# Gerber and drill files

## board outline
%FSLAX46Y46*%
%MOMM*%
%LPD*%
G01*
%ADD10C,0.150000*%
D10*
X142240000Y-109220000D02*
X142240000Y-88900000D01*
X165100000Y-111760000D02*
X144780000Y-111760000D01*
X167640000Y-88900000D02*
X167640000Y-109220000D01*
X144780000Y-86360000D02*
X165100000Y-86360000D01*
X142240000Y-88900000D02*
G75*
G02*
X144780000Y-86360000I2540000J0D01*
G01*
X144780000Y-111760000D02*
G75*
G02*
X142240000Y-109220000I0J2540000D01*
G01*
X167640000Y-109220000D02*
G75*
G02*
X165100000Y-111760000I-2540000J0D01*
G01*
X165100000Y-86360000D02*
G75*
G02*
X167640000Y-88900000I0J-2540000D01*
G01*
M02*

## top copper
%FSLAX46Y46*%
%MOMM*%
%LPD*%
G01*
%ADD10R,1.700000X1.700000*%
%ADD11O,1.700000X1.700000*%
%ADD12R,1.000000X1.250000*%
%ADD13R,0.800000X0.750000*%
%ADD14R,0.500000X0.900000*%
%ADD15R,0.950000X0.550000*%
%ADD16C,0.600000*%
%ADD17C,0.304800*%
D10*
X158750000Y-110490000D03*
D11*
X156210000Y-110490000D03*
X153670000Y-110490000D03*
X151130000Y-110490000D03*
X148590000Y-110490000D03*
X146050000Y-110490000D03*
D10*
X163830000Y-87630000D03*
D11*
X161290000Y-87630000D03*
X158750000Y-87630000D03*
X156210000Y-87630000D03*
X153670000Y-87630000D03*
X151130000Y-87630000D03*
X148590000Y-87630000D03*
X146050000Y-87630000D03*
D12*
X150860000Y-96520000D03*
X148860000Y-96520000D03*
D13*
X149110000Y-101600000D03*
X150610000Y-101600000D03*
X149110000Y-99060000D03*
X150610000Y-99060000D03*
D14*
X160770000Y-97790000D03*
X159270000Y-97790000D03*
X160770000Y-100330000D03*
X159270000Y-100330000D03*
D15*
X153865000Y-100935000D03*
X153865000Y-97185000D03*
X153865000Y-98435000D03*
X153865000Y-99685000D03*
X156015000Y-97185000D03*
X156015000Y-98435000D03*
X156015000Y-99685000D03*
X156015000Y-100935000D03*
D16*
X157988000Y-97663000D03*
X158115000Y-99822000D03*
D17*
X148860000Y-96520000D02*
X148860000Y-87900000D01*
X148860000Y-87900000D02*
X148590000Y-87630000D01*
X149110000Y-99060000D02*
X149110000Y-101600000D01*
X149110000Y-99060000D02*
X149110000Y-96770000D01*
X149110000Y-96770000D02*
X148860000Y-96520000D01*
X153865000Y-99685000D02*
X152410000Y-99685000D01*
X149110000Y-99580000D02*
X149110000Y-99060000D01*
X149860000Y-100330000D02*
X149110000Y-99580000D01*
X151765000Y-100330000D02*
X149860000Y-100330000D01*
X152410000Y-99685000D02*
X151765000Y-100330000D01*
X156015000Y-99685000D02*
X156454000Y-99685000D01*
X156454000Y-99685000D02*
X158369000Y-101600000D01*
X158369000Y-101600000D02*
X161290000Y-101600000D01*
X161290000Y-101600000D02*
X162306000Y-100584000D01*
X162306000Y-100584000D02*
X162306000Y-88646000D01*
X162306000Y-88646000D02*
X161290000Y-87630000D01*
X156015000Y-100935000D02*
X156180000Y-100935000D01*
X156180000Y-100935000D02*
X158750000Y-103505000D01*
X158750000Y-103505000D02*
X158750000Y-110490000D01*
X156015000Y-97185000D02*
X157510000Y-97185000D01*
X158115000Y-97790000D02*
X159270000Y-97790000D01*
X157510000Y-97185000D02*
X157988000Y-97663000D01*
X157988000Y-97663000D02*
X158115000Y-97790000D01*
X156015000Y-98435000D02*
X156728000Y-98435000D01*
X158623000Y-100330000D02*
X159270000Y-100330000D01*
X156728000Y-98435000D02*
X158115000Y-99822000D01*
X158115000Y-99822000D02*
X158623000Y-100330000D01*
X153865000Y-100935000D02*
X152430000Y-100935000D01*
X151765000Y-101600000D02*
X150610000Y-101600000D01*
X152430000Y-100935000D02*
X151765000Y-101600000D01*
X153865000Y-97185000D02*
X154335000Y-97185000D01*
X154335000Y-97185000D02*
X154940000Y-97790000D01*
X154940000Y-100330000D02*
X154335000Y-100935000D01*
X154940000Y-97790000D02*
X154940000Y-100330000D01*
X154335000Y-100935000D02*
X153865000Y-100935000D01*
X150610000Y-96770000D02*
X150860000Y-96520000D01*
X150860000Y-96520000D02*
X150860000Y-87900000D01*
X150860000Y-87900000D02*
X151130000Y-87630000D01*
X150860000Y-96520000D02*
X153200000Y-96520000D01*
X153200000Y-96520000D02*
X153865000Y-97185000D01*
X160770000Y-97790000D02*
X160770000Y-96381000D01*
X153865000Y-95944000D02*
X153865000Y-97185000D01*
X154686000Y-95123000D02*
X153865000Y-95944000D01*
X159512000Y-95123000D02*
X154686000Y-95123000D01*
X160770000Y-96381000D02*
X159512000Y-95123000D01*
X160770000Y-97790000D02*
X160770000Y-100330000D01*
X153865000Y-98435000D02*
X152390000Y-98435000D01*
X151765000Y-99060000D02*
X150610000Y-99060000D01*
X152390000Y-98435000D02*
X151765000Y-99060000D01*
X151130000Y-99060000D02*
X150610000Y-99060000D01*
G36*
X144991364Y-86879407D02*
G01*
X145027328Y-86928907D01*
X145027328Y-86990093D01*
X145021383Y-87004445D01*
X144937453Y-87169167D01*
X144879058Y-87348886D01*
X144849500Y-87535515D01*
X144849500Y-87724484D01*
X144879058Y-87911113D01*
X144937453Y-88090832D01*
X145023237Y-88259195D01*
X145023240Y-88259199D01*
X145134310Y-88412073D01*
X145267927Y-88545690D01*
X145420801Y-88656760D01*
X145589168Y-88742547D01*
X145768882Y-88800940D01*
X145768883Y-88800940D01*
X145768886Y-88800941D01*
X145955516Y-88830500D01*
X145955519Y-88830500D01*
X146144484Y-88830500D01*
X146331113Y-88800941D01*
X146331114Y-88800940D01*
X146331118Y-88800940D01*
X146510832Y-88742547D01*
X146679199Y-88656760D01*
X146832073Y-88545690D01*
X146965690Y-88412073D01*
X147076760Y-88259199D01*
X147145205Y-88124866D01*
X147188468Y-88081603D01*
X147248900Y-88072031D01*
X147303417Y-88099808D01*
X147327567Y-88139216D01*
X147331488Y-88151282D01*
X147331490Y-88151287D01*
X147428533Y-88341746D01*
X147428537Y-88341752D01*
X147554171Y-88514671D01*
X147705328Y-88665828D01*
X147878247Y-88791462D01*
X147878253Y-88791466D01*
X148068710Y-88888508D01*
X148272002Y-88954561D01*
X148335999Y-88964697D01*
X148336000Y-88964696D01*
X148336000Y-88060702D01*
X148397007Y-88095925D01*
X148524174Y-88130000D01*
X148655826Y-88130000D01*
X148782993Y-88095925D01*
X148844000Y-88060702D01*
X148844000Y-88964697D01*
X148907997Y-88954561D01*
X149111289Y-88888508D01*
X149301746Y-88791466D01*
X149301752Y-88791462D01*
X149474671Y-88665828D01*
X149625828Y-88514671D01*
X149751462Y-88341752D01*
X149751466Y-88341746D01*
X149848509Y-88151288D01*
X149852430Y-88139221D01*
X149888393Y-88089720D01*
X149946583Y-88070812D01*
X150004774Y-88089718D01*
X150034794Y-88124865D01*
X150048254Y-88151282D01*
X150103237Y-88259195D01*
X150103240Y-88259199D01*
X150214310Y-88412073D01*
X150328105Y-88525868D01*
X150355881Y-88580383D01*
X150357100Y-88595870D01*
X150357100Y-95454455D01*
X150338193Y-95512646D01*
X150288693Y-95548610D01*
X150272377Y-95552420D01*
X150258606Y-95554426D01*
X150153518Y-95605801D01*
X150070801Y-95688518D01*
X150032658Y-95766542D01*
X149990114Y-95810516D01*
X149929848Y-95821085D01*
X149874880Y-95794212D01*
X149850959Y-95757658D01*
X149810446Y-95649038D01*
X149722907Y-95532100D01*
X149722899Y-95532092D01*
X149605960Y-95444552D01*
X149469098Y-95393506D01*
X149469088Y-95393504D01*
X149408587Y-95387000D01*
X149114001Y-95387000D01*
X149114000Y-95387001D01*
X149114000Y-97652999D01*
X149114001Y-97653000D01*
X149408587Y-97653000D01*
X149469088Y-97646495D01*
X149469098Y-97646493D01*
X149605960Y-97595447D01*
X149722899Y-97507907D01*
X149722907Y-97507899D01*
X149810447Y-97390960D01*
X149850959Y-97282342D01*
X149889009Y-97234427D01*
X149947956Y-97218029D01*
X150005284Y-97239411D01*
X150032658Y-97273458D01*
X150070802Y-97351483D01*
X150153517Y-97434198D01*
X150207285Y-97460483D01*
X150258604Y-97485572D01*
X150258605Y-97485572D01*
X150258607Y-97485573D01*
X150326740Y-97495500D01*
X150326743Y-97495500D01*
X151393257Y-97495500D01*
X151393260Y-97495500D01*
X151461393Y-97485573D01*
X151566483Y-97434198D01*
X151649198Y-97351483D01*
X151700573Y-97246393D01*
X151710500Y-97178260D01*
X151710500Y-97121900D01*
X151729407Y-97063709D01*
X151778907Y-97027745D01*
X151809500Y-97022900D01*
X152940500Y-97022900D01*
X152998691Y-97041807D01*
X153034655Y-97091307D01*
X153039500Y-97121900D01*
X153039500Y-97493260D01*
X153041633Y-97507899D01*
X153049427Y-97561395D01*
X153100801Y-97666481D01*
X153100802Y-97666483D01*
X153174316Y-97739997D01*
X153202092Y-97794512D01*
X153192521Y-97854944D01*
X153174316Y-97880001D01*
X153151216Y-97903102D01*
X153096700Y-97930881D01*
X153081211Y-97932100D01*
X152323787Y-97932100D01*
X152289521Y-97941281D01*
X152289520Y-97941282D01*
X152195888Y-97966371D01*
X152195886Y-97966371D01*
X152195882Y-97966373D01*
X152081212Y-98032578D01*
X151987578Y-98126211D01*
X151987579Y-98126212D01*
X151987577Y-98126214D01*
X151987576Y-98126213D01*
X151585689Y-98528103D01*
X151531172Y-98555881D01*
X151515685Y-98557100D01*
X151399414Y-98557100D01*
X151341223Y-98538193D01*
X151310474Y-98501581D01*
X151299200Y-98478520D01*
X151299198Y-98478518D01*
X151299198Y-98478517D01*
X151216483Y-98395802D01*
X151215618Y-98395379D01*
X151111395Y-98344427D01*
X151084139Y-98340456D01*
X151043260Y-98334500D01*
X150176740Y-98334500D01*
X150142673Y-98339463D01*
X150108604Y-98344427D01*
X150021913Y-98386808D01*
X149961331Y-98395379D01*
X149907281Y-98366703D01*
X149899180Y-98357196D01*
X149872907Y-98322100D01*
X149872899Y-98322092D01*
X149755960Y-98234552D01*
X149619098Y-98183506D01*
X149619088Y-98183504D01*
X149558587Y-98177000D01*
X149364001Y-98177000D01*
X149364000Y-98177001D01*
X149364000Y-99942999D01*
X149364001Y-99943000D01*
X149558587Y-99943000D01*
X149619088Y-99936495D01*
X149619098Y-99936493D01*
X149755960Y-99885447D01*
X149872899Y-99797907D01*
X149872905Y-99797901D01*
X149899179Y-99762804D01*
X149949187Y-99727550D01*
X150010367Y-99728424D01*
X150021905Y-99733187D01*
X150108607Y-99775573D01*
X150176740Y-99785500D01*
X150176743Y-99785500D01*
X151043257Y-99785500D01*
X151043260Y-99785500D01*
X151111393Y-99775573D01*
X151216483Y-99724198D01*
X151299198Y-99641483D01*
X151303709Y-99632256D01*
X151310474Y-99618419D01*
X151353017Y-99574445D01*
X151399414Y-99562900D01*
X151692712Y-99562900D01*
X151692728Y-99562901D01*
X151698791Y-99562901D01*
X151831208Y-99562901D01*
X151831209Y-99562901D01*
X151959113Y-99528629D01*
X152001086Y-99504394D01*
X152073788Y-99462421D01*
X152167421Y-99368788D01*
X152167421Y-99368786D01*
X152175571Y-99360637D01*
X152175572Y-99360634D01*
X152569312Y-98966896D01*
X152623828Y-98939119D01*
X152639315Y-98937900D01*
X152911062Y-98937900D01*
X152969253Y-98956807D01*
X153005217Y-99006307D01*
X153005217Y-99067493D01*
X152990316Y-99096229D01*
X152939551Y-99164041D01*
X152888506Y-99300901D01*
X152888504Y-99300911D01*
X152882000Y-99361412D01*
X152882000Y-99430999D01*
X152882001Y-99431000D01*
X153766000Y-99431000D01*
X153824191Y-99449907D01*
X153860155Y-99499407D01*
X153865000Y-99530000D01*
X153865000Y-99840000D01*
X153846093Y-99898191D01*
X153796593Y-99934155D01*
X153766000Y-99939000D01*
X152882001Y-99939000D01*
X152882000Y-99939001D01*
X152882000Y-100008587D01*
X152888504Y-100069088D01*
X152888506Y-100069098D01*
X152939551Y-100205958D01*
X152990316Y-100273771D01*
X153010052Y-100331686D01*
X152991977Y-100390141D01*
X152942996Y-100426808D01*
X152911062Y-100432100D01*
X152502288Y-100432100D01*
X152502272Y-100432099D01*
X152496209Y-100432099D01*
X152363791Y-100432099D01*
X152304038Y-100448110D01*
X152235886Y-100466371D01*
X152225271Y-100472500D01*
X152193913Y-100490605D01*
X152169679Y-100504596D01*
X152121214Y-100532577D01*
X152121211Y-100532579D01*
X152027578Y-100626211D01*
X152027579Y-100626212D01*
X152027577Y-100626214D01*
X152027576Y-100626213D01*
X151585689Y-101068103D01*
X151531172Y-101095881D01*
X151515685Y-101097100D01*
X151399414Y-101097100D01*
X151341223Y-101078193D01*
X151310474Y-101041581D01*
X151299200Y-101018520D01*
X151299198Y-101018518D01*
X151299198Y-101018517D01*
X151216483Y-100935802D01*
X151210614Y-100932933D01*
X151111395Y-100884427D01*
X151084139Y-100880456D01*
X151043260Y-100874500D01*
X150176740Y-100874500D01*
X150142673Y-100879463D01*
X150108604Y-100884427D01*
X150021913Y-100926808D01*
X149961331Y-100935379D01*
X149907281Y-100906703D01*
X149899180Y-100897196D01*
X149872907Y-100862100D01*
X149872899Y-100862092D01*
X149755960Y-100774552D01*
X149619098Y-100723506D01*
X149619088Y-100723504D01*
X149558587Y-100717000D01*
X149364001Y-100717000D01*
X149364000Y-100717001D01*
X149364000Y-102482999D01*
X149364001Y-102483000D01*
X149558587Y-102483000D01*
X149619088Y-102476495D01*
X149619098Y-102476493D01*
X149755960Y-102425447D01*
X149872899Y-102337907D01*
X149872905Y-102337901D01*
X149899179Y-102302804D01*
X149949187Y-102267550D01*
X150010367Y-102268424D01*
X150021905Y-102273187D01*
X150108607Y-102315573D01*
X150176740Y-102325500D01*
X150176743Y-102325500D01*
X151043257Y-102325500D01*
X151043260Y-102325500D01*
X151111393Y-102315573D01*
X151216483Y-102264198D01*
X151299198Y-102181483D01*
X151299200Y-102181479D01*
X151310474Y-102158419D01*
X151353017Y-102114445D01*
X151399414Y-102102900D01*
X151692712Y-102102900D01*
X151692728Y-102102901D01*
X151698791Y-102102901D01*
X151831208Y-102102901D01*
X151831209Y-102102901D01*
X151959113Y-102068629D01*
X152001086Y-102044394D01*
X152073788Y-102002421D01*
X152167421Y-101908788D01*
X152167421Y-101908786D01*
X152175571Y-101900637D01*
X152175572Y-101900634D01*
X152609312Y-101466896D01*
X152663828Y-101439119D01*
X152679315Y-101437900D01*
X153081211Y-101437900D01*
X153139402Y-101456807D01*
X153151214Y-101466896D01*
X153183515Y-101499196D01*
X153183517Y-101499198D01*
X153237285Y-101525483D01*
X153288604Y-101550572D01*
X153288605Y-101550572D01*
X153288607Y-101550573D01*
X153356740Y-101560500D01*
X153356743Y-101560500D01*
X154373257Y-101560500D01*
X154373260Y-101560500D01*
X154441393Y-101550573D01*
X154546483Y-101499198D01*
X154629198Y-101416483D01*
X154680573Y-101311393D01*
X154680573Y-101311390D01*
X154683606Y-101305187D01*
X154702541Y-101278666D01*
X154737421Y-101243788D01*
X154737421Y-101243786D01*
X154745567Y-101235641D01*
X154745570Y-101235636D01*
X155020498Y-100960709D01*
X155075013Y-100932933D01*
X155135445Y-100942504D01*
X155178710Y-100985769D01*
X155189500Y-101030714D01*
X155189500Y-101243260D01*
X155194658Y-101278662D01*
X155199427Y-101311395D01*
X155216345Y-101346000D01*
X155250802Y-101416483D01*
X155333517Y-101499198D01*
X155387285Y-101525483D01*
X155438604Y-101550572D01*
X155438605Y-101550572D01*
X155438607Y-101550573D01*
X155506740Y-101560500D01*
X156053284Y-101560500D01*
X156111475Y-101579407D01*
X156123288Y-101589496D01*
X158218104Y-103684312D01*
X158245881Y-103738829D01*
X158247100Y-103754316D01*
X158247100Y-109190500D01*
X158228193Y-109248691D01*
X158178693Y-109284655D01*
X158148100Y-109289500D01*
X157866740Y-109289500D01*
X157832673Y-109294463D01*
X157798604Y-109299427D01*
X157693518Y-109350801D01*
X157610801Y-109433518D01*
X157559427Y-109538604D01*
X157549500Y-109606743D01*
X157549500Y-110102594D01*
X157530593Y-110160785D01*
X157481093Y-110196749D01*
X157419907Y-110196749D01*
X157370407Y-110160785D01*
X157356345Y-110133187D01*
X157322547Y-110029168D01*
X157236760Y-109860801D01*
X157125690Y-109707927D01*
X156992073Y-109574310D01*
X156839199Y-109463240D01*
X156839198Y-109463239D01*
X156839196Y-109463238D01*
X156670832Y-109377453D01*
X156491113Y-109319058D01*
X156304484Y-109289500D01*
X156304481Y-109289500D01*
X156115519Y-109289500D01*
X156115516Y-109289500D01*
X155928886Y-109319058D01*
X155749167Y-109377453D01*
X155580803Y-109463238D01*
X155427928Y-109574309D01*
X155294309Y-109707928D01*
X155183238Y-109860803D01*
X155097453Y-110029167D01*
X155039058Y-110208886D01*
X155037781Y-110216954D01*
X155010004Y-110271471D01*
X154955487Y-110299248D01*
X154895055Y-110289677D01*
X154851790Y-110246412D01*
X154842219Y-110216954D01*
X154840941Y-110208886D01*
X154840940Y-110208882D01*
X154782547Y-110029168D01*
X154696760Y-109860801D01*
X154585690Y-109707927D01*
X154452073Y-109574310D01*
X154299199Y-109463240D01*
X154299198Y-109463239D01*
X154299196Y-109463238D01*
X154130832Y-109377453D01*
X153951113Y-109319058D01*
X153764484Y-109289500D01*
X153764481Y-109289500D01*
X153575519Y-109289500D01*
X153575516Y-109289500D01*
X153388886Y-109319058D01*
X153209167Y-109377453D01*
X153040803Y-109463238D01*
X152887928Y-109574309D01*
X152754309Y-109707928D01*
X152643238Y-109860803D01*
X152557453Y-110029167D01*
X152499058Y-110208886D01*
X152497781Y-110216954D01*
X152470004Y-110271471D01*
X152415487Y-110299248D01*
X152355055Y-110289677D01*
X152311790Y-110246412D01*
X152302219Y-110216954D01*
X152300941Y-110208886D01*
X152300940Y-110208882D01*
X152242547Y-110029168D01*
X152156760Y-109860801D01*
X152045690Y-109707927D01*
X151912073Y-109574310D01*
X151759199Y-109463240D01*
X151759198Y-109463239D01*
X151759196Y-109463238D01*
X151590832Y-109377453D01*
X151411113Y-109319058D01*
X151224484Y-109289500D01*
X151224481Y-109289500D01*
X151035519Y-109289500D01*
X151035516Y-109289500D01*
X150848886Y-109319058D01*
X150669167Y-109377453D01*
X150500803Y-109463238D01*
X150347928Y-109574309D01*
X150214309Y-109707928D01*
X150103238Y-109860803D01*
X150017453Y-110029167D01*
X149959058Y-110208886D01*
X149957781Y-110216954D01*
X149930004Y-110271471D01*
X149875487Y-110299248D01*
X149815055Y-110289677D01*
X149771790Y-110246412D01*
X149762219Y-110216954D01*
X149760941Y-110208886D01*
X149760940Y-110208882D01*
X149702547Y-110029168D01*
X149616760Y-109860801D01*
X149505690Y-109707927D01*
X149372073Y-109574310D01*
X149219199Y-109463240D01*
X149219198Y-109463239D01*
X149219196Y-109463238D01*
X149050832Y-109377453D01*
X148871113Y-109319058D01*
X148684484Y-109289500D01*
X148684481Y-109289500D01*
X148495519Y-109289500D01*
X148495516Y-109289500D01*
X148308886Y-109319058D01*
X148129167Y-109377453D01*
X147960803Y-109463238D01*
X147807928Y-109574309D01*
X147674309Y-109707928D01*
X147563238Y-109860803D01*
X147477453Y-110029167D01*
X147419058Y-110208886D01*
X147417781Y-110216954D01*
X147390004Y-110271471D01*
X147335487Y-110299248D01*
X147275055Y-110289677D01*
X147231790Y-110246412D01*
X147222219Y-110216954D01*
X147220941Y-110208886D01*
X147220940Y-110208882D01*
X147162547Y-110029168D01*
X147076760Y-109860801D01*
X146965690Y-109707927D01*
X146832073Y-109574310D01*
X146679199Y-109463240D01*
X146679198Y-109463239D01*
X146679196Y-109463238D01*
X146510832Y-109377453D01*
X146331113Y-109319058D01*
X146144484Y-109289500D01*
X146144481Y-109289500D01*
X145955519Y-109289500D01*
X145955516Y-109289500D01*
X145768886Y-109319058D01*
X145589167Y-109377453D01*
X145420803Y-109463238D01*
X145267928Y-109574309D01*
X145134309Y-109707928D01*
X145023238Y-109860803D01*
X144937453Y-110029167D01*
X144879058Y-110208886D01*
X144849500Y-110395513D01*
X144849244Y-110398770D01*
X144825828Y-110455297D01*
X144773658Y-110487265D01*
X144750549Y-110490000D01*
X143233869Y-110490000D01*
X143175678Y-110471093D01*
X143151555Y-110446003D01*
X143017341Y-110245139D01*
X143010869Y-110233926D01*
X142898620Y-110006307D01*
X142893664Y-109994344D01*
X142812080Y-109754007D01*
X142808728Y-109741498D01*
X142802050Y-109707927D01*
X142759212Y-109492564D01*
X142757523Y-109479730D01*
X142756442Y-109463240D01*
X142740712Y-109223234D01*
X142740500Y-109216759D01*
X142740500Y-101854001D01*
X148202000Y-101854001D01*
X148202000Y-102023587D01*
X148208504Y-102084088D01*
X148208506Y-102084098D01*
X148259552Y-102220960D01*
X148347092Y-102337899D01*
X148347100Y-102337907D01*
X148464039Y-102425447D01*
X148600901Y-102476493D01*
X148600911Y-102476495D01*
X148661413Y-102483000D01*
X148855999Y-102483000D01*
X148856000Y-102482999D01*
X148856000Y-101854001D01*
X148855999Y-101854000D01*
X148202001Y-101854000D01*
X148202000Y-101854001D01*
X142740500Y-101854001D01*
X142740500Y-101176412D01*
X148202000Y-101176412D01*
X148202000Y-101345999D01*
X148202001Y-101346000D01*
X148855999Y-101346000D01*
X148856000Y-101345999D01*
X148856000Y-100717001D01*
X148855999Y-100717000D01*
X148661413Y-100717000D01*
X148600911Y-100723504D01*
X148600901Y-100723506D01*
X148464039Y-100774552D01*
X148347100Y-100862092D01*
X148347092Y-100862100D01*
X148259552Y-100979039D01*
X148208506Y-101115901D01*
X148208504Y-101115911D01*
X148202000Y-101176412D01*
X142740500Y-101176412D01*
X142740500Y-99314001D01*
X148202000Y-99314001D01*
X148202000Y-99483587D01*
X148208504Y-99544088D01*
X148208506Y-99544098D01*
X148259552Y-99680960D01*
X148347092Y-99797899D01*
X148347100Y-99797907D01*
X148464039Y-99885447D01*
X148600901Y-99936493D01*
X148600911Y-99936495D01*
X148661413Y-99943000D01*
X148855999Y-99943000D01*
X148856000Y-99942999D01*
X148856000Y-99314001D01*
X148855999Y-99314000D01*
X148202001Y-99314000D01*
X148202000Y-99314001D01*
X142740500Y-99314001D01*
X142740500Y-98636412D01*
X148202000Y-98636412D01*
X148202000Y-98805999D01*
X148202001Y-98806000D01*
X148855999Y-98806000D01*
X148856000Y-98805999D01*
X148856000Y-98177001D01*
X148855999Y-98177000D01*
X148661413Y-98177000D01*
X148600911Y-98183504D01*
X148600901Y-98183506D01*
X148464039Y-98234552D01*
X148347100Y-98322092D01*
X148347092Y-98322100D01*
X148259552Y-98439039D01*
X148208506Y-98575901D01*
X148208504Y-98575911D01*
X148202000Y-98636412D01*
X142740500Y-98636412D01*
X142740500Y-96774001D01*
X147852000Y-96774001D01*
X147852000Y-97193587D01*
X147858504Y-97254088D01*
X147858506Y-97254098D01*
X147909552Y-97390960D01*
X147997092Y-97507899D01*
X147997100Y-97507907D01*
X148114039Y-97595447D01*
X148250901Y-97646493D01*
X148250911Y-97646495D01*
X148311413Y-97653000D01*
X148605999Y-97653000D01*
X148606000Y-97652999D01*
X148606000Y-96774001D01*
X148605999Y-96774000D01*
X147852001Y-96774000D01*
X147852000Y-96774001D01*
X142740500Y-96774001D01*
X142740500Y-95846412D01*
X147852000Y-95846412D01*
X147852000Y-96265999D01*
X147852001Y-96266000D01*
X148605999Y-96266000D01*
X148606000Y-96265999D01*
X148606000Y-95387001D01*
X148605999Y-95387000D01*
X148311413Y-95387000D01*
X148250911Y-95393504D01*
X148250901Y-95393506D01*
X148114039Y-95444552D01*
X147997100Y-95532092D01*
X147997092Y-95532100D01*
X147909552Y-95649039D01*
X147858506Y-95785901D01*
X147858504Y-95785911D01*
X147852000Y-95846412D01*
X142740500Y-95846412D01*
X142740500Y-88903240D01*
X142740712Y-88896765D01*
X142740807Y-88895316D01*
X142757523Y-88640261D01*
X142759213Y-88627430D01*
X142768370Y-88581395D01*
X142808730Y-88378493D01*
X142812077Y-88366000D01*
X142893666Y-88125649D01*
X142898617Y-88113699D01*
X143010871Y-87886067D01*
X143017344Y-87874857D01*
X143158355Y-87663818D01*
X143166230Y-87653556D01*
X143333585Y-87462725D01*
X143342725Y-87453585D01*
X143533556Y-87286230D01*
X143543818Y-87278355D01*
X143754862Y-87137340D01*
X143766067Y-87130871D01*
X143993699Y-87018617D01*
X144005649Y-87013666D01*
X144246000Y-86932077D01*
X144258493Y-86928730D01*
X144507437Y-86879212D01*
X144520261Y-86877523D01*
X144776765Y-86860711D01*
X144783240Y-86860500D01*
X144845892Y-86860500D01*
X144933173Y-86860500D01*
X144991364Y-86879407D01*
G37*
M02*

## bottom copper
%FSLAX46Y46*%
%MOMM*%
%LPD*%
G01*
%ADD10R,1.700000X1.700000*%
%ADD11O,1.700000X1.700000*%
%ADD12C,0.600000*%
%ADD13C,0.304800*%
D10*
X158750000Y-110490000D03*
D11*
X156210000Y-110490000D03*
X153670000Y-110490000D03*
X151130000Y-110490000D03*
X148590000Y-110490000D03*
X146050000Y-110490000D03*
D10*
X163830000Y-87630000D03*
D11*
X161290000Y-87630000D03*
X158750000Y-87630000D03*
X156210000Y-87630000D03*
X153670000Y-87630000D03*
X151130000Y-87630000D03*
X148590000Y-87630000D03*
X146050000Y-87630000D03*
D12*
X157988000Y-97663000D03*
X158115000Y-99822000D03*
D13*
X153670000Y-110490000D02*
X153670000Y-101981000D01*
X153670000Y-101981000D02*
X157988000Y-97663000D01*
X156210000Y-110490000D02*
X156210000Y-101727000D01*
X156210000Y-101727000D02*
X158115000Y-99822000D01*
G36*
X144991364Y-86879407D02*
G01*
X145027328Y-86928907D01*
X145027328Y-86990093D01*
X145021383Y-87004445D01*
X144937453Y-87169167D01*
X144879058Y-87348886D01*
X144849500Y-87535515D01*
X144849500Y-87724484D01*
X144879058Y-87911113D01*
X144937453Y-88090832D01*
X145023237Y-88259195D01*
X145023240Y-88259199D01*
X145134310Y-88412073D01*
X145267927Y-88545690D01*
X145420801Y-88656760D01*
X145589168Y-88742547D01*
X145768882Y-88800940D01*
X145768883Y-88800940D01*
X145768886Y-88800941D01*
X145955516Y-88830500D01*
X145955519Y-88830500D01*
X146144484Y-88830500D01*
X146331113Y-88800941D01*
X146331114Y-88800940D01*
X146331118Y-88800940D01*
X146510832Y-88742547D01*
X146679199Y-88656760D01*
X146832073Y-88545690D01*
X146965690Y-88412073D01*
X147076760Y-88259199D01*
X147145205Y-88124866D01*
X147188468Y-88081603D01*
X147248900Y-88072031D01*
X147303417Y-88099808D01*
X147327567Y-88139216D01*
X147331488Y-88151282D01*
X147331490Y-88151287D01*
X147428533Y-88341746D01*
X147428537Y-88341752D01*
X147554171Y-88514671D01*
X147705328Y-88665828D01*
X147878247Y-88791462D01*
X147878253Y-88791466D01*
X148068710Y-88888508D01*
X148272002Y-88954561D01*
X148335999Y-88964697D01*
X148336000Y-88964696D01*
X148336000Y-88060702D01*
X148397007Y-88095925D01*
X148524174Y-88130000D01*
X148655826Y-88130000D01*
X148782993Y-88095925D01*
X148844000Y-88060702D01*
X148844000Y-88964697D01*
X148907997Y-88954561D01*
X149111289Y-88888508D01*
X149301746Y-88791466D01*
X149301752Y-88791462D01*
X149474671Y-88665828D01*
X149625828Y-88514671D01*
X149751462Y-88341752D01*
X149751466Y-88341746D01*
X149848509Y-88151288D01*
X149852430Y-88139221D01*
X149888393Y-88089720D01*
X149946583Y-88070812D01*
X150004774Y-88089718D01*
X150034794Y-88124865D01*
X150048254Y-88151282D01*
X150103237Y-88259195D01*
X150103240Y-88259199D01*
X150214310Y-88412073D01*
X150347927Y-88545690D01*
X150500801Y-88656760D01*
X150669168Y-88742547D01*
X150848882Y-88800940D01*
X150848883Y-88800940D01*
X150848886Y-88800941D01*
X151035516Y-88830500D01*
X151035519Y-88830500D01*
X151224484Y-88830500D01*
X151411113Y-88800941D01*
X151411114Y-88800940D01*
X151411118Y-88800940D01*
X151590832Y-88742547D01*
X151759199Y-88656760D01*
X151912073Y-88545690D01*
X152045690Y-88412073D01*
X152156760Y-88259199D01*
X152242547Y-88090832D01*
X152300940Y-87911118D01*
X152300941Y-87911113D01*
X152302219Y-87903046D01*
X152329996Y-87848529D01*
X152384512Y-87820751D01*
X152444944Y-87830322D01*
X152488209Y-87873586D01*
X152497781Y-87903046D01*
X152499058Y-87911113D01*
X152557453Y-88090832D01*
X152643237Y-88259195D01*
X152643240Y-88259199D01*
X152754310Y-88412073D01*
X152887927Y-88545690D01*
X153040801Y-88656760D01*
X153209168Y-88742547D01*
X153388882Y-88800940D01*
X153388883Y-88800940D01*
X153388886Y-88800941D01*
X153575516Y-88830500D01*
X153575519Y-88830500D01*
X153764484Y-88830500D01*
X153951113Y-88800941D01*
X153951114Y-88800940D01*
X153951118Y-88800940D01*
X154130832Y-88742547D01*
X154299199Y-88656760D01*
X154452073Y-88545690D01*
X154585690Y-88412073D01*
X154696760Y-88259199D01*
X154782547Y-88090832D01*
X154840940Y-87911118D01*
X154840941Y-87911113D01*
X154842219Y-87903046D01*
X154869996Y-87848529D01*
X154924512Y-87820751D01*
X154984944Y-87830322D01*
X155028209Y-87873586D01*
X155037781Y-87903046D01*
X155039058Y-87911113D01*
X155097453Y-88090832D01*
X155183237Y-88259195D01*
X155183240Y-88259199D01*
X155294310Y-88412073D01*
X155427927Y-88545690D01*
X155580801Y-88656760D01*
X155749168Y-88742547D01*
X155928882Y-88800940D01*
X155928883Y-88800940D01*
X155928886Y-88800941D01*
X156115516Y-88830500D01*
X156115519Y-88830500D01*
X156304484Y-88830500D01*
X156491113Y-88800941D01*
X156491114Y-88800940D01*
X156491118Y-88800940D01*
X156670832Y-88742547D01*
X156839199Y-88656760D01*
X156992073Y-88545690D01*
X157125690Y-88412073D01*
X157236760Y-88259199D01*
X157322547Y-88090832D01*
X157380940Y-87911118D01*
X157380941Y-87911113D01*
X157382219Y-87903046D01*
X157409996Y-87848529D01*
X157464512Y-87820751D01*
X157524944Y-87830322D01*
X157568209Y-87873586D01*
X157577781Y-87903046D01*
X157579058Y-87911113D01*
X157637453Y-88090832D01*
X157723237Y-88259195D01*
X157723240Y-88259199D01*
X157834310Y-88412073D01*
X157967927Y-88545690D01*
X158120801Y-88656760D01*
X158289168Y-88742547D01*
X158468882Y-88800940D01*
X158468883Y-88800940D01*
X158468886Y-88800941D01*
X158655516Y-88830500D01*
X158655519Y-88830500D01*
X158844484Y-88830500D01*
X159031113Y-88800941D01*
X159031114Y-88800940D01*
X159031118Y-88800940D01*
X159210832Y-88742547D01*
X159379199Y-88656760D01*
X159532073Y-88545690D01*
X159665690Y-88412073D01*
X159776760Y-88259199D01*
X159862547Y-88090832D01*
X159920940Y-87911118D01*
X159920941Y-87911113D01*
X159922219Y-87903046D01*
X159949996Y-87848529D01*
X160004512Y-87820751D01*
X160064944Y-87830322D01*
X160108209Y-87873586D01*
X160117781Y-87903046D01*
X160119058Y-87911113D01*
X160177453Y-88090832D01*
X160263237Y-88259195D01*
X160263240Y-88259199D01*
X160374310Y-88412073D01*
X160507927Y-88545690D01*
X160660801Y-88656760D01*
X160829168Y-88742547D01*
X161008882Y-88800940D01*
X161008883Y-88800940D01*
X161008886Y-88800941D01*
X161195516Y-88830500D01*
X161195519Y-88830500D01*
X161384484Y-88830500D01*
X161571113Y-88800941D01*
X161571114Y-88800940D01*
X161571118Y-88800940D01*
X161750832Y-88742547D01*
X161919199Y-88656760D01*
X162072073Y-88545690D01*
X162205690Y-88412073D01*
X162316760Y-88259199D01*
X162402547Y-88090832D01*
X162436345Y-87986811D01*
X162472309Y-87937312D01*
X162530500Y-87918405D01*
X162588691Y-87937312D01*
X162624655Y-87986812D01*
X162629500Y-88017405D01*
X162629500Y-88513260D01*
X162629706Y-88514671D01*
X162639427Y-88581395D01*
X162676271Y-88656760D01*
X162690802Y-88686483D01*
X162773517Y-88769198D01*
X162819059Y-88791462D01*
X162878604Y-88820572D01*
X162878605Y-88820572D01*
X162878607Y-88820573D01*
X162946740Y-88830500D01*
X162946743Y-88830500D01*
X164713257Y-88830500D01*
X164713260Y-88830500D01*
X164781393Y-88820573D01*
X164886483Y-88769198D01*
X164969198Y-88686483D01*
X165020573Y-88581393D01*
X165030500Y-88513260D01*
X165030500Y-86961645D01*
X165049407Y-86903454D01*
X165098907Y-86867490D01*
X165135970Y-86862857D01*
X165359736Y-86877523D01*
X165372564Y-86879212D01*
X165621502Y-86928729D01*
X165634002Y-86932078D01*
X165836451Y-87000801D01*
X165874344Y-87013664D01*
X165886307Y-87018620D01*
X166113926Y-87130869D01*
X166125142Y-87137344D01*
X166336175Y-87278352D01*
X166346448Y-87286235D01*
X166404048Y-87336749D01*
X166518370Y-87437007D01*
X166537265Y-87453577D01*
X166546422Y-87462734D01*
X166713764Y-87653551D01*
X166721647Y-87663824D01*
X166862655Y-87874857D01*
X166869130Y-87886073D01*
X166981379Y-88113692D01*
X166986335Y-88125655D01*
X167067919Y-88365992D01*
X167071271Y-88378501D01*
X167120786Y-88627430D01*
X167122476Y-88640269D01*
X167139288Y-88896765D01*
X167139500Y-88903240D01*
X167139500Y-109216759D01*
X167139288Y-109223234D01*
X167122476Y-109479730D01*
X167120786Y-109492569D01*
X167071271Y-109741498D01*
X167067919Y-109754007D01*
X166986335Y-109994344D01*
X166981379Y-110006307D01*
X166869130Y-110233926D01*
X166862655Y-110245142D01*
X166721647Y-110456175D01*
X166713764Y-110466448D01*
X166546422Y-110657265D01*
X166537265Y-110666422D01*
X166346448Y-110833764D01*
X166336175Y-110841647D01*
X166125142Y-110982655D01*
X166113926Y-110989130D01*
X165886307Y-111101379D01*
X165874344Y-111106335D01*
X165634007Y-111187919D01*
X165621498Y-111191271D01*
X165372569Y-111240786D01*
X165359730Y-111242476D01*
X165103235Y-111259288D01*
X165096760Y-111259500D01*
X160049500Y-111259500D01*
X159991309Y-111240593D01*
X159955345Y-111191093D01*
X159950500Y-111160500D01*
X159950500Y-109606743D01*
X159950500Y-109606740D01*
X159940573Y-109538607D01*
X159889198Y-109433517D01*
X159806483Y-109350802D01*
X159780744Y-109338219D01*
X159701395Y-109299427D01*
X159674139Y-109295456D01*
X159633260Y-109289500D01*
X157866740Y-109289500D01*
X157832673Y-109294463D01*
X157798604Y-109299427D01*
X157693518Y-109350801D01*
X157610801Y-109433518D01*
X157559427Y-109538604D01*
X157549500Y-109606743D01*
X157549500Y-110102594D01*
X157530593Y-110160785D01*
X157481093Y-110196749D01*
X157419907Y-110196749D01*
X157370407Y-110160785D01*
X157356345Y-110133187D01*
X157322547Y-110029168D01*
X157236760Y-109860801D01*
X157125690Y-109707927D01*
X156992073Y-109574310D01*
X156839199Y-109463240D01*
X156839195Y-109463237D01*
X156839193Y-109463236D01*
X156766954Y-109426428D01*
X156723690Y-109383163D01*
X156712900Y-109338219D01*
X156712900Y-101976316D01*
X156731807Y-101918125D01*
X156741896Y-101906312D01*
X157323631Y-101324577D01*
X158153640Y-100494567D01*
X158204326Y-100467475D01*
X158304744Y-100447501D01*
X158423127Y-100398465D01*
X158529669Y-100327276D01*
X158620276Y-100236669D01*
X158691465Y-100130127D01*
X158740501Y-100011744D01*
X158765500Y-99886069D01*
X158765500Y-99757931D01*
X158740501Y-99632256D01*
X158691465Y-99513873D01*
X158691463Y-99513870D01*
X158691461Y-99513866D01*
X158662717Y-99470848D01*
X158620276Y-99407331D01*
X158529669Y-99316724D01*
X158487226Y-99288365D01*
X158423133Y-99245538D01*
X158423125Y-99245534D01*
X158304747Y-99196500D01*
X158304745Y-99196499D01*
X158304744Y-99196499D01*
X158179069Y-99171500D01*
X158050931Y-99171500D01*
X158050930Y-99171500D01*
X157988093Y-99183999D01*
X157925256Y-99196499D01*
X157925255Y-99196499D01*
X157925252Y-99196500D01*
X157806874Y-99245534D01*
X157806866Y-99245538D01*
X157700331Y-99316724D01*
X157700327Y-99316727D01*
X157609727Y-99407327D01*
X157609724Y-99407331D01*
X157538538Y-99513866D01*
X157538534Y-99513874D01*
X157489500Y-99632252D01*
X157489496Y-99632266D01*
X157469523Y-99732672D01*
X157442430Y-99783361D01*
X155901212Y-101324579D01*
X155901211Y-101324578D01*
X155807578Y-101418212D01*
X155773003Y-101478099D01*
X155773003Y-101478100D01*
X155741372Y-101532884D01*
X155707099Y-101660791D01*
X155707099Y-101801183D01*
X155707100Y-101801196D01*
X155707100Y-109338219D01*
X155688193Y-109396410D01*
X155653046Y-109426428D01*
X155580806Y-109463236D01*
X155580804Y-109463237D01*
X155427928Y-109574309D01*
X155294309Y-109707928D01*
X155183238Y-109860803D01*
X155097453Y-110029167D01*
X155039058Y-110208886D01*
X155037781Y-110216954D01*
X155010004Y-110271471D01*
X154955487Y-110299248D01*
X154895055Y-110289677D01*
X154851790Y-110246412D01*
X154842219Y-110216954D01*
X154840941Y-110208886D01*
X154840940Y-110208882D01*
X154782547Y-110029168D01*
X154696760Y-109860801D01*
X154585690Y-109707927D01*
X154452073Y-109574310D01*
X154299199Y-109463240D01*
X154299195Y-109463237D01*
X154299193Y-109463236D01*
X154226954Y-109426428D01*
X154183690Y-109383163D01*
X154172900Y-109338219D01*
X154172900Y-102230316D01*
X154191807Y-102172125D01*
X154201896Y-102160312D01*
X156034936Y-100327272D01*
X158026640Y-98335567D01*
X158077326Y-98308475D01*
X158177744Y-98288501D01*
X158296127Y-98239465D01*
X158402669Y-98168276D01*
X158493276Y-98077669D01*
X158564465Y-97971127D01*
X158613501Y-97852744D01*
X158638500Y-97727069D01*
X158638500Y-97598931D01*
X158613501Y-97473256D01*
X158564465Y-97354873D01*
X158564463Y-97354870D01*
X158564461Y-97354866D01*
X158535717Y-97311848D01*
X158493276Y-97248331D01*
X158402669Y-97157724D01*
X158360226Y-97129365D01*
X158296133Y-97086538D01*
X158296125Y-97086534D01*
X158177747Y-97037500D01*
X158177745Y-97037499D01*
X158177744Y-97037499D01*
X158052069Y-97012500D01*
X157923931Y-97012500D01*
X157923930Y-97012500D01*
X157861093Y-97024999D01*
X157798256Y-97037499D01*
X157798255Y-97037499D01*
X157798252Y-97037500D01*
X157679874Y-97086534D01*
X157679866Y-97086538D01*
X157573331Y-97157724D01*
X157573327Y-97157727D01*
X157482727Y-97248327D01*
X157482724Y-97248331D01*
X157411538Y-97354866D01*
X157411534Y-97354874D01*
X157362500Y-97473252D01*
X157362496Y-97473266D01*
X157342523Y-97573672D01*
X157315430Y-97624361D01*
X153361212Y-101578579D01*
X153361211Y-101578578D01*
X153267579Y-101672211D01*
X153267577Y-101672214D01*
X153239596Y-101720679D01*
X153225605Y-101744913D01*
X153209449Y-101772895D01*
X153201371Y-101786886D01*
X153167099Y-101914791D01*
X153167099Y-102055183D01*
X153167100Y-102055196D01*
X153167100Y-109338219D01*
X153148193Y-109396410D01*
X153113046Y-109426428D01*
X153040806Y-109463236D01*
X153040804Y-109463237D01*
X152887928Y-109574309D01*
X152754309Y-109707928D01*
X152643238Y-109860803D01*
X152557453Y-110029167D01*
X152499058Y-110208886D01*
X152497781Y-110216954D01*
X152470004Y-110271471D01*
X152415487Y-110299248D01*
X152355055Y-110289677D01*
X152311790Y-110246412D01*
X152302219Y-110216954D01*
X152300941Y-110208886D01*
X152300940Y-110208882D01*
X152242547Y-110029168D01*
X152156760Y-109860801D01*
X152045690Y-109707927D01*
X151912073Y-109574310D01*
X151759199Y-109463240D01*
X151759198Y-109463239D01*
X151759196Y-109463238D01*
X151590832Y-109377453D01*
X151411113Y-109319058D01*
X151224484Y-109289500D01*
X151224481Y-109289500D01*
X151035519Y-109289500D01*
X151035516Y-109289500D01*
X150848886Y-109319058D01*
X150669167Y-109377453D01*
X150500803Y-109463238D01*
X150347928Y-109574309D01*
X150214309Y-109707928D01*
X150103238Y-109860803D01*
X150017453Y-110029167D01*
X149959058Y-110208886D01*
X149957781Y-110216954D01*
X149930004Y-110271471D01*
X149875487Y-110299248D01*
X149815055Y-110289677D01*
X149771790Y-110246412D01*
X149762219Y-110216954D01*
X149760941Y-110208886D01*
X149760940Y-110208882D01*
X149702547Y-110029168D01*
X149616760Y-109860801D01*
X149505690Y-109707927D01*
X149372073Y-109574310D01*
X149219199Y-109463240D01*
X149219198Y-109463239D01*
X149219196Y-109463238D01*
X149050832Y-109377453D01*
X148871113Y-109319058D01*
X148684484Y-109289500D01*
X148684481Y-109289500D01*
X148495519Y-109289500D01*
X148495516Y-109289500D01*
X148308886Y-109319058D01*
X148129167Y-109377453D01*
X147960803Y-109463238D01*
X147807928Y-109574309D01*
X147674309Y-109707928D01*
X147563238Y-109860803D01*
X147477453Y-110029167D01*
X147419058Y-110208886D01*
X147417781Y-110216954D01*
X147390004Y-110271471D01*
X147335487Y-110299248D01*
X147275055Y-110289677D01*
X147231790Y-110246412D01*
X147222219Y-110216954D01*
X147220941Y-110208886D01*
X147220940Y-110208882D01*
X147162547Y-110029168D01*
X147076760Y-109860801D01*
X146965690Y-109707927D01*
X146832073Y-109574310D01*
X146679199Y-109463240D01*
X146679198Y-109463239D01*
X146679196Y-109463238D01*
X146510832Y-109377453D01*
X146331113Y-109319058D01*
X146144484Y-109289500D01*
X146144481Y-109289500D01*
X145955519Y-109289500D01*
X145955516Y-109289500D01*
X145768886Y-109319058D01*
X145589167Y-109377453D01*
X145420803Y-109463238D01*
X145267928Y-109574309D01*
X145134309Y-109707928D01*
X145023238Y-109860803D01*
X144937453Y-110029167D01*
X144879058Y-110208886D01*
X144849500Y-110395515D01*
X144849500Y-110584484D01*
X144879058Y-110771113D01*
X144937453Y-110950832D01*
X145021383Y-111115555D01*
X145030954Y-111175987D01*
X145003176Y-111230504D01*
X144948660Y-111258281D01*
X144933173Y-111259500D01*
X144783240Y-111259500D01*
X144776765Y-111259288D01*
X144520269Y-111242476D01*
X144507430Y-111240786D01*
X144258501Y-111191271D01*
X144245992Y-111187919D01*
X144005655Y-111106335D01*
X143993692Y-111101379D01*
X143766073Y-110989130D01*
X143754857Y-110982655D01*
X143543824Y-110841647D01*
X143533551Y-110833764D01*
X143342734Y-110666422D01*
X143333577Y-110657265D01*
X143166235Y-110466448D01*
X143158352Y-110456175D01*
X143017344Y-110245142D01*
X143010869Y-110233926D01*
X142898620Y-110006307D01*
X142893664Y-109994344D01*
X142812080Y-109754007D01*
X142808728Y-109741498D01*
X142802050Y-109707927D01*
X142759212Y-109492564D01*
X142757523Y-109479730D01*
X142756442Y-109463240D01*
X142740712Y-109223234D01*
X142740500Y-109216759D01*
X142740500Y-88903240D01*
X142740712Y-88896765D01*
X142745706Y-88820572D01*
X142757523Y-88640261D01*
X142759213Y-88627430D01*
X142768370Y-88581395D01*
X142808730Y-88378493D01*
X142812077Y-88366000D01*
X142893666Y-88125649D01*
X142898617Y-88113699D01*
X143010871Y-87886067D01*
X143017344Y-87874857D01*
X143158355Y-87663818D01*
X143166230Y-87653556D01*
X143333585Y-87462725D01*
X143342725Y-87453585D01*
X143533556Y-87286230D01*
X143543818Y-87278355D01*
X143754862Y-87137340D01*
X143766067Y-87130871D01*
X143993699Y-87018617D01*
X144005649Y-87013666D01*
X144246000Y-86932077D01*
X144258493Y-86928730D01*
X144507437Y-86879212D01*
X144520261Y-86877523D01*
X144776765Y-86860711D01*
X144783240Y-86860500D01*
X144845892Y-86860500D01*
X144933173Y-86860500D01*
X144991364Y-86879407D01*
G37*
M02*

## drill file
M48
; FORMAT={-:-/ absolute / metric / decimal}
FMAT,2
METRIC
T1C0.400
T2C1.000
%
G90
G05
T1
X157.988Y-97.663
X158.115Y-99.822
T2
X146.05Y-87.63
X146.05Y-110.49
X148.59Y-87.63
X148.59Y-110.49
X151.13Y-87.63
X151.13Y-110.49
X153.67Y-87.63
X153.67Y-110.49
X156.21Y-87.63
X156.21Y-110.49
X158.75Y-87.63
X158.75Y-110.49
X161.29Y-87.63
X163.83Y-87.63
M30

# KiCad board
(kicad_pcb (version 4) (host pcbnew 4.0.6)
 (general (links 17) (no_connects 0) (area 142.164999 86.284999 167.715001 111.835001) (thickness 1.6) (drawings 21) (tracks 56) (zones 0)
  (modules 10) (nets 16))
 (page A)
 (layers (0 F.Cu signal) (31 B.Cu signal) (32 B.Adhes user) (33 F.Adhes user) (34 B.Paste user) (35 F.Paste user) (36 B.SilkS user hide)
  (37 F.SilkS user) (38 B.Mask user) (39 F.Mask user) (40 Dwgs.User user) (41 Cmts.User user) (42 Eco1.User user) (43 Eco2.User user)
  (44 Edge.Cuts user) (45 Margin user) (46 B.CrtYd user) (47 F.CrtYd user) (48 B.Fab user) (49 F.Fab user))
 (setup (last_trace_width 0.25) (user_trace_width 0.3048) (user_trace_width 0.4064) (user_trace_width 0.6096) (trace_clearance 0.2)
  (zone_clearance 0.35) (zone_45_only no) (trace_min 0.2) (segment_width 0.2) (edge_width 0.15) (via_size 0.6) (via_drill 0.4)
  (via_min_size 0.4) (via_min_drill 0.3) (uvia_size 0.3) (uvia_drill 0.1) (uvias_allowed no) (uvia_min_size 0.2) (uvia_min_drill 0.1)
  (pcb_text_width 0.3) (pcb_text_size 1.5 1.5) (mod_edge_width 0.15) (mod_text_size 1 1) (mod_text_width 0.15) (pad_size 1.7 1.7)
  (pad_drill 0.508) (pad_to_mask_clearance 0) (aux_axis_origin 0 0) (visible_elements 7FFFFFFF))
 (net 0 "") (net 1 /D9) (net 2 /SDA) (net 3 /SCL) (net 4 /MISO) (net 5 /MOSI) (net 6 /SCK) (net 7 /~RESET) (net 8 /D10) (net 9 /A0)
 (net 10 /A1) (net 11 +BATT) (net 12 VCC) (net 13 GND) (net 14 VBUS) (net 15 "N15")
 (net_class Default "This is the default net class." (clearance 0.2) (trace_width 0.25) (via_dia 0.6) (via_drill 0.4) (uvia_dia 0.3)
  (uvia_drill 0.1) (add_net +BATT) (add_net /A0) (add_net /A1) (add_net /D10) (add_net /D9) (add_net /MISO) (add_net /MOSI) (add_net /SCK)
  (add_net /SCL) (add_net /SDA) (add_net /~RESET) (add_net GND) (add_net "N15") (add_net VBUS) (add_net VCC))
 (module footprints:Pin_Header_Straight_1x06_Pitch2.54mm (layer F.Cu) (at 158.75 110.49 270)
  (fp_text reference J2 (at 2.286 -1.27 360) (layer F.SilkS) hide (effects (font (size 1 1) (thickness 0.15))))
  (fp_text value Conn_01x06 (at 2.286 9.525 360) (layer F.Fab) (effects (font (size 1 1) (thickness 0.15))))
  (pad 1 thru_hole rect (at 0 0 270) (size 1.7 1.7) (drill 1) (layers *.Cu *.Mask) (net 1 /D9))
  (pad 2 thru_hole oval (at 0 2.54 270) (size 1.7 1.7) (drill 1) (layers *.Cu *.Mask) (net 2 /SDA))
  (pad 3 thru_hole oval (at 0 5.08 270) (size 1.7 1.7) (drill 1) (layers *.Cu *.Mask) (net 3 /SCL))
  (pad 4 thru_hole oval (at 0 7.62 270) (size 1.7 1.7) (drill 1) (layers *.Cu *.Mask) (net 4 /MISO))
  (pad 5 thru_hole oval (at 0 10.16 270) (size 1.7 1.7) (drill 1) (layers *.Cu *.Mask) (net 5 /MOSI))
  (pad 6 thru_hole oval (at 0 12.7 270) (size 1.7 1.7) (drill 1) (layers *.Cu *.Mask) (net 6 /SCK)))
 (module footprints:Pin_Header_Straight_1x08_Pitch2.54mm (layer F.Cu) (at 163.83 87.63 270)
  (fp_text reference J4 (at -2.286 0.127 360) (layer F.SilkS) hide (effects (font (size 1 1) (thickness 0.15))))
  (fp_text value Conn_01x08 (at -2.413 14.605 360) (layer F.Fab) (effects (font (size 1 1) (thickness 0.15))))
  (pad 1 thru_hole rect (at 0 0 270) (size 1.7 1.7) (drill 1) (layers *.Cu *.Mask) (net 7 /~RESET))
  (pad 2 thru_hole oval (at 0 2.54 270) (size 1.7 1.7) (drill 1) (layers *.Cu *.Mask) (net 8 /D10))
  (pad 3 thru_hole oval (at 0 5.08 270) (size 1.7 1.7) (drill 1) (layers *.Cu *.Mask) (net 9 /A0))
  (pad 4 thru_hole oval (at 0 7.62 270) (size 1.7 1.7) (drill 1) (layers *.Cu *.Mask) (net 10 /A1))
  (pad 5 thru_hole oval (at 0 10.16 270) (size 1.7 1.7) (drill 1) (layers *.Cu *.Mask) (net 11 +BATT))
  (pad 6 thru_hole oval (at 0 12.7 270) (size 1.7 1.7) (drill 1) (layers *.Cu *.Mask) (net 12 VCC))
  (pad 7 thru_hole oval (at 0 15.24 270) (size 1.7 1.7) (drill 1) (layers *.Cu *.Mask) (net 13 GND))
  (pad 8 thru_hole oval (at 0 17.78 270) (size 1.7 1.7) (drill 1) (layers *.Cu *.Mask) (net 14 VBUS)))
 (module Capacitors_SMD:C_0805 (layer F.Cu) (at 149.86 96.52 180)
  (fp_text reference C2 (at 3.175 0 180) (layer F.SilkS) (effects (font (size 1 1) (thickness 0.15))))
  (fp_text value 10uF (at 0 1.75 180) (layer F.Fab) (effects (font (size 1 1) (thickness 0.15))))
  (pad 1 smd rect (at -1 0 180) (size 1 1.25) (layers F.Cu F.Paste F.Mask) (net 12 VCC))
  (pad 2 smd rect (at 1 0 180) (size 1 1.25) (layers F.Cu F.Paste F.Mask) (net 13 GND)))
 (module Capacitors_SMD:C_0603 (layer F.Cu) (at 149.86 101.6 180)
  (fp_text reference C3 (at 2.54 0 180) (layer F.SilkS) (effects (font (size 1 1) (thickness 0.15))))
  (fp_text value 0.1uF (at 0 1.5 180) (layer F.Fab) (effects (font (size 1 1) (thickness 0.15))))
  (pad 2 smd rect (at 0.75 0 180) (size 0.8 0.75) (layers F.Cu F.Paste F.Mask) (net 13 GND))
  (pad 1 smd rect (at -0.75 0 180) (size 0.8 0.75) (layers F.Cu F.Paste F.Mask) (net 12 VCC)))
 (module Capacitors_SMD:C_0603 (layer F.Cu) (at 149.86 99.06 180)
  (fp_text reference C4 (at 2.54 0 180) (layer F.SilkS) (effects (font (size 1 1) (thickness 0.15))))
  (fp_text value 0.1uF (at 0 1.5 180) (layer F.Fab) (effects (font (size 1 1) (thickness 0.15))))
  (pad 2 smd rect (at 0.75 0 180) (size 0.8 0.75) (layers F.Cu F.Paste F.Mask) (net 13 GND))
  (pad 1 smd rect (at -0.75 0 180) (size 0.8 0.75) (layers F.Cu F.Paste F.Mask) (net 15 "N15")))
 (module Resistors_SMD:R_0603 (layer F.Cu) (at 160.02 97.79 180)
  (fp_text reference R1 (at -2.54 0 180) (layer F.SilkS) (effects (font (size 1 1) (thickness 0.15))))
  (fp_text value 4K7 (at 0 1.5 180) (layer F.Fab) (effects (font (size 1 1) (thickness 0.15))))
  (pad 1 smd rect (at -0.75 0 180) (size 0.5 0.9) (layers F.Cu F.Paste F.Mask) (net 12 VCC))
  (pad 2 smd rect (at 0.75 0 180) (size 0.5 0.9) (layers F.Cu F.Paste F.Mask) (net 3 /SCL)))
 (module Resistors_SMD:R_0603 (layer F.Cu) (at 160.02 100.33 180)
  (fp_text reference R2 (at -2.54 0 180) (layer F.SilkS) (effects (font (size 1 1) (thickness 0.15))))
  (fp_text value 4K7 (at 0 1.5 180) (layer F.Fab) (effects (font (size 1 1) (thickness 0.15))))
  (pad 1 smd rect (at -0.75 0 180) (size 0.5 0.9) (layers F.Cu F.Paste F.Mask) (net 12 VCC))
  (pad 2 smd rect (at 0.75 0 180) (size 0.5 0.9) (layers F.Cu F.Paste F.Mask) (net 2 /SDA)))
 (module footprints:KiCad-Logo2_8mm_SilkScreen (layer B.Cu) (at 158.115 104.14 180)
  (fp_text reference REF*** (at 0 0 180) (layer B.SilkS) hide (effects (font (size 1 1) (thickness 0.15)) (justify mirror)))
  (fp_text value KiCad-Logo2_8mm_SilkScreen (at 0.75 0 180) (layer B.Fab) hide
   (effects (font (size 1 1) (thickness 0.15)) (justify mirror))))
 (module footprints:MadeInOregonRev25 (layer F.Cu) (at 145.923 100.584)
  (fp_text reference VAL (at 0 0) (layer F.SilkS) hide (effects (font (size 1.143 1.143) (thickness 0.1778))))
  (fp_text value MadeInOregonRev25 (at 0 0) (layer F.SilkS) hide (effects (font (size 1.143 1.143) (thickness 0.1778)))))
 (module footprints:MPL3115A (layer F.Cu) (at 154.94 99.06)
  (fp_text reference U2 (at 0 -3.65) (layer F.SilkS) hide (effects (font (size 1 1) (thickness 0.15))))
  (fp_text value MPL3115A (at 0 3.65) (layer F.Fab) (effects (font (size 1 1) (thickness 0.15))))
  (pad 4 smd rect (at -1.075 1.875) (size 0.95 0.55) (layers F.Cu F.Paste F.Mask) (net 12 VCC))
  (pad 1 smd rect (at -1.075 -1.875) (size 0.95 0.55) (layers F.Cu F.Paste F.Mask) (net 12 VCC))
  (pad 2 smd rect (at -1.075 -0.625) (size 0.95 0.55) (layers F.Cu F.Paste F.Mask) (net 15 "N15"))
  (pad 3 smd rect (at -1.075 0.625) (size 0.95 0.55) (layers F.Cu F.Paste F.Mask) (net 13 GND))
  (pad 8 smd rect (at 1.075 -1.875) (size 0.95 0.55) (layers F.Cu F.Paste F.Mask) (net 3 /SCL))
  (pad 7 smd rect (at 1.075 -0.625) (size 0.95 0.55) (layers F.Cu F.Paste F.Mask) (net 2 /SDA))
  (pad 6 smd rect (at 1.075 0.625) (size 0.95 0.55) (layers F.Cu F.Paste F.Mask) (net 8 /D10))
  (pad 5 smd rect (at 1.075 1.875) (size 0.95 0.55) (layers F.Cu F.Paste F.Mask) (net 1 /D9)))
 (gr_line (start 142.24 109.22) (end 142.24 88.9) (angle 90) (layer Edge.Cuts) (width 0.15))
 (gr_line (start 165.1 111.76) (end 144.78 111.76) (angle 90) (layer Edge.Cuts) (width 0.15))
 (gr_line (start 167.64 88.9) (end 167.64 109.22) (angle 90) (layer Edge.Cuts) (width 0.15))
 (gr_line (start 144.78 86.36) (end 165.1 86.36) (angle 90) (layer Edge.Cuts) (width 0.15))
 (gr_arc (start 144.78 88.9) (end 142.24 88.9) (angle 90) (layer Edge.Cuts) (width 0.15))
 (gr_arc (start 144.78 109.22) (end 144.78 111.76) (angle 90) (layer Edge.Cuts) (width 0.15))
 (gr_arc (start 165.1 109.22) (end 167.64 109.22) (angle 90) (layer Edge.Cuts) (width 0.15))
 (gr_arc (start 165.1 88.9) (end 165.1 86.36) (angle 90) (layer Edge.Cuts) (width 0.15))
 (segment (start 148.86 96.52) (end 148.86 87.9) (width 0.3048) (layer F.Cu) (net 13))
 (segment (start 148.86 87.9) (end 148.59 87.63) (width 0.3048) (layer F.Cu) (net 13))
 (segment (start 149.11 99.06) (end 149.11 101.6) (width 0.3048) (layer F.Cu) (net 13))
 (segment (start 149.11 99.06) (end 149.11 96.77) (width 0.3048) (layer F.Cu) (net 13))
 (segment (start 149.11 96.77) (end 148.86 96.52) (width 0.3048) (layer F.Cu) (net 13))
 (segment (start 153.865 99.685) (end 152.41 99.685) (width 0.3048) (layer F.Cu) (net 13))
 (segment (start 149.11 99.58) (end 149.11 99.06) (width 0.3048) (layer F.Cu) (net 13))
 (segment (start 149.86 100.33) (end 149.11 99.58) (width 0.3048) (layer F.Cu) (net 13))
 (segment (start 151.765 100.33) (end 149.86 100.33) (width 0.3048) (layer F.Cu) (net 13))
 (segment (start 152.41 99.685) (end 151.765 100.33) (width 0.3048) (layer F.Cu) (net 13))
 (segment (start 156.015 99.685) (end 156.454 99.685) (width 0.3048) (layer F.Cu) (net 8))
 (segment (start 156.454 99.685) (end 158.369 101.6) (width 0.3048) (layer F.Cu) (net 8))
 (segment (start 158.369 101.6) (end 161.29 101.6) (width 0.3048) (layer F.Cu) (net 8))
 (segment (start 161.29 101.6) (end 162.306 100.584) (width 0.3048) (layer F.Cu) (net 8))
 (segment (start 162.306 100.584) (end 162.306 88.646) (width 0.3048) (layer F.Cu) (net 8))
 (segment (start 162.306 88.646) (end 161.29 87.63) (width 0.3048) (layer F.Cu) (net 8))
 (segment (start 156.015 100.935) (end 156.18 100.935) (width 0.3048) (layer F.Cu) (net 1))
 (segment (start 156.18 100.935) (end 158.75 103.505) (width 0.3048) (layer F.Cu) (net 1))
 (segment (start 158.75 103.505) (end 158.75 110.49) (width 0.3048) (layer F.Cu) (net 1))
 (via (at 157.988 97.663) (size 0.6) (drill 0.4) (layers F.Cu B.Cu) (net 3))
 (segment (start 153.67 110.49) (end 153.67 101.981) (width 0.3048) (layer B.Cu) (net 3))
 (segment (start 153.67 101.981) (end 157.988 97.663) (width 0.3048) (layer B.Cu) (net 3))
 (segment (start 156.015 97.185) (end 157.51 97.185) (width 0.3048) (layer F.Cu) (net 3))
 (segment (start 158.115 97.79) (end 159.27 97.79) (width 0.3048) (layer F.Cu) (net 3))
 (segment (start 157.51 97.185) (end 157.988 97.663) (width 0.3048) (layer F.Cu) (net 3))
 (segment (start 157.988 97.663) (end 158.115 97.79) (width 0.3048) (layer F.Cu) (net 3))
 (via (at 158.115 99.822) (size 0.6) (drill 0.4) (layers F.Cu B.Cu) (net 2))
 (segment (start 156.21 110.49) (end 156.21 101.727) (width 0.3048) (layer B.Cu) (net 2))
 (segment (start 156.21 101.727) (end 158.115 99.822) (width 0.3048) (layer B.Cu) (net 2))
 (segment (start 156.015 98.435) (end 156.728 98.435) (width 0.3048) (layer F.Cu) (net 2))
 (segment (start 158.623 100.33) (end 159.27 100.33) (width 0.3048) (layer F.Cu) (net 2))
 (segment (start 156.728 98.435) (end 158.115 99.822) (width 0.3048) (layer F.Cu) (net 2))
 (segment (start 158.115 99.822) (end 158.623 100.33) (width 0.3048) (layer F.Cu) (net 2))
 (segment (start 153.865 100.935) (end 152.43 100.935) (width 0.3048) (layer F.Cu) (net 12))
 (segment (start 151.765 101.6) (end 150.61 101.6) (width 0.3048) (layer F.Cu) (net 12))
 (segment (start 152.43 100.935) (end 151.765 101.6) (width 0.3048) (layer F.Cu) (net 12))
 (segment (start 153.865 97.185) (end 154.335 97.185) (width 0.3048) (layer F.Cu) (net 12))
 (segment (start 154.335 97.185) (end 154.94 97.79) (width 0.3048) (layer F.Cu) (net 12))
 (segment (start 154.94 100.33) (end 154.335 100.935) (width 0.3048) (layer F.Cu) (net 12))
 (segment (start 154.94 97.79) (end 154.94 100.33) (width 0.3048) (layer F.Cu) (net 12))
 (segment (start 154.335 100.935) (end 153.865 100.935) (width 0.3048) (layer F.Cu) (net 12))
 (segment (start 150.61 96.77) (end 150.86 96.52) (width 0.3048) (layer F.Cu) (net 12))
 (segment (start 150.86 96.52) (end 150.86 87.9) (width 0.3048) (layer F.Cu) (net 12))
 (segment (start 150.86 87.9) (end 151.13 87.63) (width 0.3048) (layer F.Cu) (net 12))
 (segment (start 150.86 96.52) (end 153.2 96.52) (width 0.3048) (layer F.Cu) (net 12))
 (segment (start 153.2 96.52) (end 153.865 97.185) (width 0.3048) (layer F.Cu) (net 12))
 (segment (start 160.77 97.79) (end 160.77 96.381) (width 0.3048) (layer F.Cu) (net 12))
 (segment (start 153.865 95.944) (end 153.865 97.185) (width 0.3048) (layer F.Cu) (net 12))
 (segment (start 154.686 95.123) (end 153.865 95.944) (width 0.3048) (layer F.Cu) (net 12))
 (segment (start 159.512 95.123) (end 154.686 95.123) (width 0.3048) (layer F.Cu) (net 12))
 (segment (start 160.77 96.381) (end 159.512 95.123) (width 0.3048) (layer F.Cu) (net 12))
 (segment (start 160.77 97.79) (end 160.77 100.33) (width 0.3048) (layer F.Cu) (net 12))
 (segment (start 153.865 98.435) (end 152.39 98.435) (width 0.3048) (layer F.Cu) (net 15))
 (segment (start 151.765 99.06) (end 150.61 99.06) (width 0.3048) (layer F.Cu) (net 15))
 (segment (start 152.39 98.435) (end 151.765 99.06) (width 0.3048) (layer F.Cu) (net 15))
 (segment (start 151.13 99.06) (end 150.61 99.06) (width 0.3048) (layer F.Cu) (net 15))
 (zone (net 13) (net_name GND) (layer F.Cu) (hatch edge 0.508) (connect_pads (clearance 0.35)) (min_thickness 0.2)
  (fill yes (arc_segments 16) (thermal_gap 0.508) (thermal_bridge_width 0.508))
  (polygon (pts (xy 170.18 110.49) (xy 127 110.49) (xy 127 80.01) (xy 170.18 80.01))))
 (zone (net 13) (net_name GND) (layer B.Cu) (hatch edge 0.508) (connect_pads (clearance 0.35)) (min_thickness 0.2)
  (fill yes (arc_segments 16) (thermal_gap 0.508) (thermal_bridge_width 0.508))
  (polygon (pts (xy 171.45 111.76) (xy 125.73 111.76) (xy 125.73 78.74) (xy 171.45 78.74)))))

